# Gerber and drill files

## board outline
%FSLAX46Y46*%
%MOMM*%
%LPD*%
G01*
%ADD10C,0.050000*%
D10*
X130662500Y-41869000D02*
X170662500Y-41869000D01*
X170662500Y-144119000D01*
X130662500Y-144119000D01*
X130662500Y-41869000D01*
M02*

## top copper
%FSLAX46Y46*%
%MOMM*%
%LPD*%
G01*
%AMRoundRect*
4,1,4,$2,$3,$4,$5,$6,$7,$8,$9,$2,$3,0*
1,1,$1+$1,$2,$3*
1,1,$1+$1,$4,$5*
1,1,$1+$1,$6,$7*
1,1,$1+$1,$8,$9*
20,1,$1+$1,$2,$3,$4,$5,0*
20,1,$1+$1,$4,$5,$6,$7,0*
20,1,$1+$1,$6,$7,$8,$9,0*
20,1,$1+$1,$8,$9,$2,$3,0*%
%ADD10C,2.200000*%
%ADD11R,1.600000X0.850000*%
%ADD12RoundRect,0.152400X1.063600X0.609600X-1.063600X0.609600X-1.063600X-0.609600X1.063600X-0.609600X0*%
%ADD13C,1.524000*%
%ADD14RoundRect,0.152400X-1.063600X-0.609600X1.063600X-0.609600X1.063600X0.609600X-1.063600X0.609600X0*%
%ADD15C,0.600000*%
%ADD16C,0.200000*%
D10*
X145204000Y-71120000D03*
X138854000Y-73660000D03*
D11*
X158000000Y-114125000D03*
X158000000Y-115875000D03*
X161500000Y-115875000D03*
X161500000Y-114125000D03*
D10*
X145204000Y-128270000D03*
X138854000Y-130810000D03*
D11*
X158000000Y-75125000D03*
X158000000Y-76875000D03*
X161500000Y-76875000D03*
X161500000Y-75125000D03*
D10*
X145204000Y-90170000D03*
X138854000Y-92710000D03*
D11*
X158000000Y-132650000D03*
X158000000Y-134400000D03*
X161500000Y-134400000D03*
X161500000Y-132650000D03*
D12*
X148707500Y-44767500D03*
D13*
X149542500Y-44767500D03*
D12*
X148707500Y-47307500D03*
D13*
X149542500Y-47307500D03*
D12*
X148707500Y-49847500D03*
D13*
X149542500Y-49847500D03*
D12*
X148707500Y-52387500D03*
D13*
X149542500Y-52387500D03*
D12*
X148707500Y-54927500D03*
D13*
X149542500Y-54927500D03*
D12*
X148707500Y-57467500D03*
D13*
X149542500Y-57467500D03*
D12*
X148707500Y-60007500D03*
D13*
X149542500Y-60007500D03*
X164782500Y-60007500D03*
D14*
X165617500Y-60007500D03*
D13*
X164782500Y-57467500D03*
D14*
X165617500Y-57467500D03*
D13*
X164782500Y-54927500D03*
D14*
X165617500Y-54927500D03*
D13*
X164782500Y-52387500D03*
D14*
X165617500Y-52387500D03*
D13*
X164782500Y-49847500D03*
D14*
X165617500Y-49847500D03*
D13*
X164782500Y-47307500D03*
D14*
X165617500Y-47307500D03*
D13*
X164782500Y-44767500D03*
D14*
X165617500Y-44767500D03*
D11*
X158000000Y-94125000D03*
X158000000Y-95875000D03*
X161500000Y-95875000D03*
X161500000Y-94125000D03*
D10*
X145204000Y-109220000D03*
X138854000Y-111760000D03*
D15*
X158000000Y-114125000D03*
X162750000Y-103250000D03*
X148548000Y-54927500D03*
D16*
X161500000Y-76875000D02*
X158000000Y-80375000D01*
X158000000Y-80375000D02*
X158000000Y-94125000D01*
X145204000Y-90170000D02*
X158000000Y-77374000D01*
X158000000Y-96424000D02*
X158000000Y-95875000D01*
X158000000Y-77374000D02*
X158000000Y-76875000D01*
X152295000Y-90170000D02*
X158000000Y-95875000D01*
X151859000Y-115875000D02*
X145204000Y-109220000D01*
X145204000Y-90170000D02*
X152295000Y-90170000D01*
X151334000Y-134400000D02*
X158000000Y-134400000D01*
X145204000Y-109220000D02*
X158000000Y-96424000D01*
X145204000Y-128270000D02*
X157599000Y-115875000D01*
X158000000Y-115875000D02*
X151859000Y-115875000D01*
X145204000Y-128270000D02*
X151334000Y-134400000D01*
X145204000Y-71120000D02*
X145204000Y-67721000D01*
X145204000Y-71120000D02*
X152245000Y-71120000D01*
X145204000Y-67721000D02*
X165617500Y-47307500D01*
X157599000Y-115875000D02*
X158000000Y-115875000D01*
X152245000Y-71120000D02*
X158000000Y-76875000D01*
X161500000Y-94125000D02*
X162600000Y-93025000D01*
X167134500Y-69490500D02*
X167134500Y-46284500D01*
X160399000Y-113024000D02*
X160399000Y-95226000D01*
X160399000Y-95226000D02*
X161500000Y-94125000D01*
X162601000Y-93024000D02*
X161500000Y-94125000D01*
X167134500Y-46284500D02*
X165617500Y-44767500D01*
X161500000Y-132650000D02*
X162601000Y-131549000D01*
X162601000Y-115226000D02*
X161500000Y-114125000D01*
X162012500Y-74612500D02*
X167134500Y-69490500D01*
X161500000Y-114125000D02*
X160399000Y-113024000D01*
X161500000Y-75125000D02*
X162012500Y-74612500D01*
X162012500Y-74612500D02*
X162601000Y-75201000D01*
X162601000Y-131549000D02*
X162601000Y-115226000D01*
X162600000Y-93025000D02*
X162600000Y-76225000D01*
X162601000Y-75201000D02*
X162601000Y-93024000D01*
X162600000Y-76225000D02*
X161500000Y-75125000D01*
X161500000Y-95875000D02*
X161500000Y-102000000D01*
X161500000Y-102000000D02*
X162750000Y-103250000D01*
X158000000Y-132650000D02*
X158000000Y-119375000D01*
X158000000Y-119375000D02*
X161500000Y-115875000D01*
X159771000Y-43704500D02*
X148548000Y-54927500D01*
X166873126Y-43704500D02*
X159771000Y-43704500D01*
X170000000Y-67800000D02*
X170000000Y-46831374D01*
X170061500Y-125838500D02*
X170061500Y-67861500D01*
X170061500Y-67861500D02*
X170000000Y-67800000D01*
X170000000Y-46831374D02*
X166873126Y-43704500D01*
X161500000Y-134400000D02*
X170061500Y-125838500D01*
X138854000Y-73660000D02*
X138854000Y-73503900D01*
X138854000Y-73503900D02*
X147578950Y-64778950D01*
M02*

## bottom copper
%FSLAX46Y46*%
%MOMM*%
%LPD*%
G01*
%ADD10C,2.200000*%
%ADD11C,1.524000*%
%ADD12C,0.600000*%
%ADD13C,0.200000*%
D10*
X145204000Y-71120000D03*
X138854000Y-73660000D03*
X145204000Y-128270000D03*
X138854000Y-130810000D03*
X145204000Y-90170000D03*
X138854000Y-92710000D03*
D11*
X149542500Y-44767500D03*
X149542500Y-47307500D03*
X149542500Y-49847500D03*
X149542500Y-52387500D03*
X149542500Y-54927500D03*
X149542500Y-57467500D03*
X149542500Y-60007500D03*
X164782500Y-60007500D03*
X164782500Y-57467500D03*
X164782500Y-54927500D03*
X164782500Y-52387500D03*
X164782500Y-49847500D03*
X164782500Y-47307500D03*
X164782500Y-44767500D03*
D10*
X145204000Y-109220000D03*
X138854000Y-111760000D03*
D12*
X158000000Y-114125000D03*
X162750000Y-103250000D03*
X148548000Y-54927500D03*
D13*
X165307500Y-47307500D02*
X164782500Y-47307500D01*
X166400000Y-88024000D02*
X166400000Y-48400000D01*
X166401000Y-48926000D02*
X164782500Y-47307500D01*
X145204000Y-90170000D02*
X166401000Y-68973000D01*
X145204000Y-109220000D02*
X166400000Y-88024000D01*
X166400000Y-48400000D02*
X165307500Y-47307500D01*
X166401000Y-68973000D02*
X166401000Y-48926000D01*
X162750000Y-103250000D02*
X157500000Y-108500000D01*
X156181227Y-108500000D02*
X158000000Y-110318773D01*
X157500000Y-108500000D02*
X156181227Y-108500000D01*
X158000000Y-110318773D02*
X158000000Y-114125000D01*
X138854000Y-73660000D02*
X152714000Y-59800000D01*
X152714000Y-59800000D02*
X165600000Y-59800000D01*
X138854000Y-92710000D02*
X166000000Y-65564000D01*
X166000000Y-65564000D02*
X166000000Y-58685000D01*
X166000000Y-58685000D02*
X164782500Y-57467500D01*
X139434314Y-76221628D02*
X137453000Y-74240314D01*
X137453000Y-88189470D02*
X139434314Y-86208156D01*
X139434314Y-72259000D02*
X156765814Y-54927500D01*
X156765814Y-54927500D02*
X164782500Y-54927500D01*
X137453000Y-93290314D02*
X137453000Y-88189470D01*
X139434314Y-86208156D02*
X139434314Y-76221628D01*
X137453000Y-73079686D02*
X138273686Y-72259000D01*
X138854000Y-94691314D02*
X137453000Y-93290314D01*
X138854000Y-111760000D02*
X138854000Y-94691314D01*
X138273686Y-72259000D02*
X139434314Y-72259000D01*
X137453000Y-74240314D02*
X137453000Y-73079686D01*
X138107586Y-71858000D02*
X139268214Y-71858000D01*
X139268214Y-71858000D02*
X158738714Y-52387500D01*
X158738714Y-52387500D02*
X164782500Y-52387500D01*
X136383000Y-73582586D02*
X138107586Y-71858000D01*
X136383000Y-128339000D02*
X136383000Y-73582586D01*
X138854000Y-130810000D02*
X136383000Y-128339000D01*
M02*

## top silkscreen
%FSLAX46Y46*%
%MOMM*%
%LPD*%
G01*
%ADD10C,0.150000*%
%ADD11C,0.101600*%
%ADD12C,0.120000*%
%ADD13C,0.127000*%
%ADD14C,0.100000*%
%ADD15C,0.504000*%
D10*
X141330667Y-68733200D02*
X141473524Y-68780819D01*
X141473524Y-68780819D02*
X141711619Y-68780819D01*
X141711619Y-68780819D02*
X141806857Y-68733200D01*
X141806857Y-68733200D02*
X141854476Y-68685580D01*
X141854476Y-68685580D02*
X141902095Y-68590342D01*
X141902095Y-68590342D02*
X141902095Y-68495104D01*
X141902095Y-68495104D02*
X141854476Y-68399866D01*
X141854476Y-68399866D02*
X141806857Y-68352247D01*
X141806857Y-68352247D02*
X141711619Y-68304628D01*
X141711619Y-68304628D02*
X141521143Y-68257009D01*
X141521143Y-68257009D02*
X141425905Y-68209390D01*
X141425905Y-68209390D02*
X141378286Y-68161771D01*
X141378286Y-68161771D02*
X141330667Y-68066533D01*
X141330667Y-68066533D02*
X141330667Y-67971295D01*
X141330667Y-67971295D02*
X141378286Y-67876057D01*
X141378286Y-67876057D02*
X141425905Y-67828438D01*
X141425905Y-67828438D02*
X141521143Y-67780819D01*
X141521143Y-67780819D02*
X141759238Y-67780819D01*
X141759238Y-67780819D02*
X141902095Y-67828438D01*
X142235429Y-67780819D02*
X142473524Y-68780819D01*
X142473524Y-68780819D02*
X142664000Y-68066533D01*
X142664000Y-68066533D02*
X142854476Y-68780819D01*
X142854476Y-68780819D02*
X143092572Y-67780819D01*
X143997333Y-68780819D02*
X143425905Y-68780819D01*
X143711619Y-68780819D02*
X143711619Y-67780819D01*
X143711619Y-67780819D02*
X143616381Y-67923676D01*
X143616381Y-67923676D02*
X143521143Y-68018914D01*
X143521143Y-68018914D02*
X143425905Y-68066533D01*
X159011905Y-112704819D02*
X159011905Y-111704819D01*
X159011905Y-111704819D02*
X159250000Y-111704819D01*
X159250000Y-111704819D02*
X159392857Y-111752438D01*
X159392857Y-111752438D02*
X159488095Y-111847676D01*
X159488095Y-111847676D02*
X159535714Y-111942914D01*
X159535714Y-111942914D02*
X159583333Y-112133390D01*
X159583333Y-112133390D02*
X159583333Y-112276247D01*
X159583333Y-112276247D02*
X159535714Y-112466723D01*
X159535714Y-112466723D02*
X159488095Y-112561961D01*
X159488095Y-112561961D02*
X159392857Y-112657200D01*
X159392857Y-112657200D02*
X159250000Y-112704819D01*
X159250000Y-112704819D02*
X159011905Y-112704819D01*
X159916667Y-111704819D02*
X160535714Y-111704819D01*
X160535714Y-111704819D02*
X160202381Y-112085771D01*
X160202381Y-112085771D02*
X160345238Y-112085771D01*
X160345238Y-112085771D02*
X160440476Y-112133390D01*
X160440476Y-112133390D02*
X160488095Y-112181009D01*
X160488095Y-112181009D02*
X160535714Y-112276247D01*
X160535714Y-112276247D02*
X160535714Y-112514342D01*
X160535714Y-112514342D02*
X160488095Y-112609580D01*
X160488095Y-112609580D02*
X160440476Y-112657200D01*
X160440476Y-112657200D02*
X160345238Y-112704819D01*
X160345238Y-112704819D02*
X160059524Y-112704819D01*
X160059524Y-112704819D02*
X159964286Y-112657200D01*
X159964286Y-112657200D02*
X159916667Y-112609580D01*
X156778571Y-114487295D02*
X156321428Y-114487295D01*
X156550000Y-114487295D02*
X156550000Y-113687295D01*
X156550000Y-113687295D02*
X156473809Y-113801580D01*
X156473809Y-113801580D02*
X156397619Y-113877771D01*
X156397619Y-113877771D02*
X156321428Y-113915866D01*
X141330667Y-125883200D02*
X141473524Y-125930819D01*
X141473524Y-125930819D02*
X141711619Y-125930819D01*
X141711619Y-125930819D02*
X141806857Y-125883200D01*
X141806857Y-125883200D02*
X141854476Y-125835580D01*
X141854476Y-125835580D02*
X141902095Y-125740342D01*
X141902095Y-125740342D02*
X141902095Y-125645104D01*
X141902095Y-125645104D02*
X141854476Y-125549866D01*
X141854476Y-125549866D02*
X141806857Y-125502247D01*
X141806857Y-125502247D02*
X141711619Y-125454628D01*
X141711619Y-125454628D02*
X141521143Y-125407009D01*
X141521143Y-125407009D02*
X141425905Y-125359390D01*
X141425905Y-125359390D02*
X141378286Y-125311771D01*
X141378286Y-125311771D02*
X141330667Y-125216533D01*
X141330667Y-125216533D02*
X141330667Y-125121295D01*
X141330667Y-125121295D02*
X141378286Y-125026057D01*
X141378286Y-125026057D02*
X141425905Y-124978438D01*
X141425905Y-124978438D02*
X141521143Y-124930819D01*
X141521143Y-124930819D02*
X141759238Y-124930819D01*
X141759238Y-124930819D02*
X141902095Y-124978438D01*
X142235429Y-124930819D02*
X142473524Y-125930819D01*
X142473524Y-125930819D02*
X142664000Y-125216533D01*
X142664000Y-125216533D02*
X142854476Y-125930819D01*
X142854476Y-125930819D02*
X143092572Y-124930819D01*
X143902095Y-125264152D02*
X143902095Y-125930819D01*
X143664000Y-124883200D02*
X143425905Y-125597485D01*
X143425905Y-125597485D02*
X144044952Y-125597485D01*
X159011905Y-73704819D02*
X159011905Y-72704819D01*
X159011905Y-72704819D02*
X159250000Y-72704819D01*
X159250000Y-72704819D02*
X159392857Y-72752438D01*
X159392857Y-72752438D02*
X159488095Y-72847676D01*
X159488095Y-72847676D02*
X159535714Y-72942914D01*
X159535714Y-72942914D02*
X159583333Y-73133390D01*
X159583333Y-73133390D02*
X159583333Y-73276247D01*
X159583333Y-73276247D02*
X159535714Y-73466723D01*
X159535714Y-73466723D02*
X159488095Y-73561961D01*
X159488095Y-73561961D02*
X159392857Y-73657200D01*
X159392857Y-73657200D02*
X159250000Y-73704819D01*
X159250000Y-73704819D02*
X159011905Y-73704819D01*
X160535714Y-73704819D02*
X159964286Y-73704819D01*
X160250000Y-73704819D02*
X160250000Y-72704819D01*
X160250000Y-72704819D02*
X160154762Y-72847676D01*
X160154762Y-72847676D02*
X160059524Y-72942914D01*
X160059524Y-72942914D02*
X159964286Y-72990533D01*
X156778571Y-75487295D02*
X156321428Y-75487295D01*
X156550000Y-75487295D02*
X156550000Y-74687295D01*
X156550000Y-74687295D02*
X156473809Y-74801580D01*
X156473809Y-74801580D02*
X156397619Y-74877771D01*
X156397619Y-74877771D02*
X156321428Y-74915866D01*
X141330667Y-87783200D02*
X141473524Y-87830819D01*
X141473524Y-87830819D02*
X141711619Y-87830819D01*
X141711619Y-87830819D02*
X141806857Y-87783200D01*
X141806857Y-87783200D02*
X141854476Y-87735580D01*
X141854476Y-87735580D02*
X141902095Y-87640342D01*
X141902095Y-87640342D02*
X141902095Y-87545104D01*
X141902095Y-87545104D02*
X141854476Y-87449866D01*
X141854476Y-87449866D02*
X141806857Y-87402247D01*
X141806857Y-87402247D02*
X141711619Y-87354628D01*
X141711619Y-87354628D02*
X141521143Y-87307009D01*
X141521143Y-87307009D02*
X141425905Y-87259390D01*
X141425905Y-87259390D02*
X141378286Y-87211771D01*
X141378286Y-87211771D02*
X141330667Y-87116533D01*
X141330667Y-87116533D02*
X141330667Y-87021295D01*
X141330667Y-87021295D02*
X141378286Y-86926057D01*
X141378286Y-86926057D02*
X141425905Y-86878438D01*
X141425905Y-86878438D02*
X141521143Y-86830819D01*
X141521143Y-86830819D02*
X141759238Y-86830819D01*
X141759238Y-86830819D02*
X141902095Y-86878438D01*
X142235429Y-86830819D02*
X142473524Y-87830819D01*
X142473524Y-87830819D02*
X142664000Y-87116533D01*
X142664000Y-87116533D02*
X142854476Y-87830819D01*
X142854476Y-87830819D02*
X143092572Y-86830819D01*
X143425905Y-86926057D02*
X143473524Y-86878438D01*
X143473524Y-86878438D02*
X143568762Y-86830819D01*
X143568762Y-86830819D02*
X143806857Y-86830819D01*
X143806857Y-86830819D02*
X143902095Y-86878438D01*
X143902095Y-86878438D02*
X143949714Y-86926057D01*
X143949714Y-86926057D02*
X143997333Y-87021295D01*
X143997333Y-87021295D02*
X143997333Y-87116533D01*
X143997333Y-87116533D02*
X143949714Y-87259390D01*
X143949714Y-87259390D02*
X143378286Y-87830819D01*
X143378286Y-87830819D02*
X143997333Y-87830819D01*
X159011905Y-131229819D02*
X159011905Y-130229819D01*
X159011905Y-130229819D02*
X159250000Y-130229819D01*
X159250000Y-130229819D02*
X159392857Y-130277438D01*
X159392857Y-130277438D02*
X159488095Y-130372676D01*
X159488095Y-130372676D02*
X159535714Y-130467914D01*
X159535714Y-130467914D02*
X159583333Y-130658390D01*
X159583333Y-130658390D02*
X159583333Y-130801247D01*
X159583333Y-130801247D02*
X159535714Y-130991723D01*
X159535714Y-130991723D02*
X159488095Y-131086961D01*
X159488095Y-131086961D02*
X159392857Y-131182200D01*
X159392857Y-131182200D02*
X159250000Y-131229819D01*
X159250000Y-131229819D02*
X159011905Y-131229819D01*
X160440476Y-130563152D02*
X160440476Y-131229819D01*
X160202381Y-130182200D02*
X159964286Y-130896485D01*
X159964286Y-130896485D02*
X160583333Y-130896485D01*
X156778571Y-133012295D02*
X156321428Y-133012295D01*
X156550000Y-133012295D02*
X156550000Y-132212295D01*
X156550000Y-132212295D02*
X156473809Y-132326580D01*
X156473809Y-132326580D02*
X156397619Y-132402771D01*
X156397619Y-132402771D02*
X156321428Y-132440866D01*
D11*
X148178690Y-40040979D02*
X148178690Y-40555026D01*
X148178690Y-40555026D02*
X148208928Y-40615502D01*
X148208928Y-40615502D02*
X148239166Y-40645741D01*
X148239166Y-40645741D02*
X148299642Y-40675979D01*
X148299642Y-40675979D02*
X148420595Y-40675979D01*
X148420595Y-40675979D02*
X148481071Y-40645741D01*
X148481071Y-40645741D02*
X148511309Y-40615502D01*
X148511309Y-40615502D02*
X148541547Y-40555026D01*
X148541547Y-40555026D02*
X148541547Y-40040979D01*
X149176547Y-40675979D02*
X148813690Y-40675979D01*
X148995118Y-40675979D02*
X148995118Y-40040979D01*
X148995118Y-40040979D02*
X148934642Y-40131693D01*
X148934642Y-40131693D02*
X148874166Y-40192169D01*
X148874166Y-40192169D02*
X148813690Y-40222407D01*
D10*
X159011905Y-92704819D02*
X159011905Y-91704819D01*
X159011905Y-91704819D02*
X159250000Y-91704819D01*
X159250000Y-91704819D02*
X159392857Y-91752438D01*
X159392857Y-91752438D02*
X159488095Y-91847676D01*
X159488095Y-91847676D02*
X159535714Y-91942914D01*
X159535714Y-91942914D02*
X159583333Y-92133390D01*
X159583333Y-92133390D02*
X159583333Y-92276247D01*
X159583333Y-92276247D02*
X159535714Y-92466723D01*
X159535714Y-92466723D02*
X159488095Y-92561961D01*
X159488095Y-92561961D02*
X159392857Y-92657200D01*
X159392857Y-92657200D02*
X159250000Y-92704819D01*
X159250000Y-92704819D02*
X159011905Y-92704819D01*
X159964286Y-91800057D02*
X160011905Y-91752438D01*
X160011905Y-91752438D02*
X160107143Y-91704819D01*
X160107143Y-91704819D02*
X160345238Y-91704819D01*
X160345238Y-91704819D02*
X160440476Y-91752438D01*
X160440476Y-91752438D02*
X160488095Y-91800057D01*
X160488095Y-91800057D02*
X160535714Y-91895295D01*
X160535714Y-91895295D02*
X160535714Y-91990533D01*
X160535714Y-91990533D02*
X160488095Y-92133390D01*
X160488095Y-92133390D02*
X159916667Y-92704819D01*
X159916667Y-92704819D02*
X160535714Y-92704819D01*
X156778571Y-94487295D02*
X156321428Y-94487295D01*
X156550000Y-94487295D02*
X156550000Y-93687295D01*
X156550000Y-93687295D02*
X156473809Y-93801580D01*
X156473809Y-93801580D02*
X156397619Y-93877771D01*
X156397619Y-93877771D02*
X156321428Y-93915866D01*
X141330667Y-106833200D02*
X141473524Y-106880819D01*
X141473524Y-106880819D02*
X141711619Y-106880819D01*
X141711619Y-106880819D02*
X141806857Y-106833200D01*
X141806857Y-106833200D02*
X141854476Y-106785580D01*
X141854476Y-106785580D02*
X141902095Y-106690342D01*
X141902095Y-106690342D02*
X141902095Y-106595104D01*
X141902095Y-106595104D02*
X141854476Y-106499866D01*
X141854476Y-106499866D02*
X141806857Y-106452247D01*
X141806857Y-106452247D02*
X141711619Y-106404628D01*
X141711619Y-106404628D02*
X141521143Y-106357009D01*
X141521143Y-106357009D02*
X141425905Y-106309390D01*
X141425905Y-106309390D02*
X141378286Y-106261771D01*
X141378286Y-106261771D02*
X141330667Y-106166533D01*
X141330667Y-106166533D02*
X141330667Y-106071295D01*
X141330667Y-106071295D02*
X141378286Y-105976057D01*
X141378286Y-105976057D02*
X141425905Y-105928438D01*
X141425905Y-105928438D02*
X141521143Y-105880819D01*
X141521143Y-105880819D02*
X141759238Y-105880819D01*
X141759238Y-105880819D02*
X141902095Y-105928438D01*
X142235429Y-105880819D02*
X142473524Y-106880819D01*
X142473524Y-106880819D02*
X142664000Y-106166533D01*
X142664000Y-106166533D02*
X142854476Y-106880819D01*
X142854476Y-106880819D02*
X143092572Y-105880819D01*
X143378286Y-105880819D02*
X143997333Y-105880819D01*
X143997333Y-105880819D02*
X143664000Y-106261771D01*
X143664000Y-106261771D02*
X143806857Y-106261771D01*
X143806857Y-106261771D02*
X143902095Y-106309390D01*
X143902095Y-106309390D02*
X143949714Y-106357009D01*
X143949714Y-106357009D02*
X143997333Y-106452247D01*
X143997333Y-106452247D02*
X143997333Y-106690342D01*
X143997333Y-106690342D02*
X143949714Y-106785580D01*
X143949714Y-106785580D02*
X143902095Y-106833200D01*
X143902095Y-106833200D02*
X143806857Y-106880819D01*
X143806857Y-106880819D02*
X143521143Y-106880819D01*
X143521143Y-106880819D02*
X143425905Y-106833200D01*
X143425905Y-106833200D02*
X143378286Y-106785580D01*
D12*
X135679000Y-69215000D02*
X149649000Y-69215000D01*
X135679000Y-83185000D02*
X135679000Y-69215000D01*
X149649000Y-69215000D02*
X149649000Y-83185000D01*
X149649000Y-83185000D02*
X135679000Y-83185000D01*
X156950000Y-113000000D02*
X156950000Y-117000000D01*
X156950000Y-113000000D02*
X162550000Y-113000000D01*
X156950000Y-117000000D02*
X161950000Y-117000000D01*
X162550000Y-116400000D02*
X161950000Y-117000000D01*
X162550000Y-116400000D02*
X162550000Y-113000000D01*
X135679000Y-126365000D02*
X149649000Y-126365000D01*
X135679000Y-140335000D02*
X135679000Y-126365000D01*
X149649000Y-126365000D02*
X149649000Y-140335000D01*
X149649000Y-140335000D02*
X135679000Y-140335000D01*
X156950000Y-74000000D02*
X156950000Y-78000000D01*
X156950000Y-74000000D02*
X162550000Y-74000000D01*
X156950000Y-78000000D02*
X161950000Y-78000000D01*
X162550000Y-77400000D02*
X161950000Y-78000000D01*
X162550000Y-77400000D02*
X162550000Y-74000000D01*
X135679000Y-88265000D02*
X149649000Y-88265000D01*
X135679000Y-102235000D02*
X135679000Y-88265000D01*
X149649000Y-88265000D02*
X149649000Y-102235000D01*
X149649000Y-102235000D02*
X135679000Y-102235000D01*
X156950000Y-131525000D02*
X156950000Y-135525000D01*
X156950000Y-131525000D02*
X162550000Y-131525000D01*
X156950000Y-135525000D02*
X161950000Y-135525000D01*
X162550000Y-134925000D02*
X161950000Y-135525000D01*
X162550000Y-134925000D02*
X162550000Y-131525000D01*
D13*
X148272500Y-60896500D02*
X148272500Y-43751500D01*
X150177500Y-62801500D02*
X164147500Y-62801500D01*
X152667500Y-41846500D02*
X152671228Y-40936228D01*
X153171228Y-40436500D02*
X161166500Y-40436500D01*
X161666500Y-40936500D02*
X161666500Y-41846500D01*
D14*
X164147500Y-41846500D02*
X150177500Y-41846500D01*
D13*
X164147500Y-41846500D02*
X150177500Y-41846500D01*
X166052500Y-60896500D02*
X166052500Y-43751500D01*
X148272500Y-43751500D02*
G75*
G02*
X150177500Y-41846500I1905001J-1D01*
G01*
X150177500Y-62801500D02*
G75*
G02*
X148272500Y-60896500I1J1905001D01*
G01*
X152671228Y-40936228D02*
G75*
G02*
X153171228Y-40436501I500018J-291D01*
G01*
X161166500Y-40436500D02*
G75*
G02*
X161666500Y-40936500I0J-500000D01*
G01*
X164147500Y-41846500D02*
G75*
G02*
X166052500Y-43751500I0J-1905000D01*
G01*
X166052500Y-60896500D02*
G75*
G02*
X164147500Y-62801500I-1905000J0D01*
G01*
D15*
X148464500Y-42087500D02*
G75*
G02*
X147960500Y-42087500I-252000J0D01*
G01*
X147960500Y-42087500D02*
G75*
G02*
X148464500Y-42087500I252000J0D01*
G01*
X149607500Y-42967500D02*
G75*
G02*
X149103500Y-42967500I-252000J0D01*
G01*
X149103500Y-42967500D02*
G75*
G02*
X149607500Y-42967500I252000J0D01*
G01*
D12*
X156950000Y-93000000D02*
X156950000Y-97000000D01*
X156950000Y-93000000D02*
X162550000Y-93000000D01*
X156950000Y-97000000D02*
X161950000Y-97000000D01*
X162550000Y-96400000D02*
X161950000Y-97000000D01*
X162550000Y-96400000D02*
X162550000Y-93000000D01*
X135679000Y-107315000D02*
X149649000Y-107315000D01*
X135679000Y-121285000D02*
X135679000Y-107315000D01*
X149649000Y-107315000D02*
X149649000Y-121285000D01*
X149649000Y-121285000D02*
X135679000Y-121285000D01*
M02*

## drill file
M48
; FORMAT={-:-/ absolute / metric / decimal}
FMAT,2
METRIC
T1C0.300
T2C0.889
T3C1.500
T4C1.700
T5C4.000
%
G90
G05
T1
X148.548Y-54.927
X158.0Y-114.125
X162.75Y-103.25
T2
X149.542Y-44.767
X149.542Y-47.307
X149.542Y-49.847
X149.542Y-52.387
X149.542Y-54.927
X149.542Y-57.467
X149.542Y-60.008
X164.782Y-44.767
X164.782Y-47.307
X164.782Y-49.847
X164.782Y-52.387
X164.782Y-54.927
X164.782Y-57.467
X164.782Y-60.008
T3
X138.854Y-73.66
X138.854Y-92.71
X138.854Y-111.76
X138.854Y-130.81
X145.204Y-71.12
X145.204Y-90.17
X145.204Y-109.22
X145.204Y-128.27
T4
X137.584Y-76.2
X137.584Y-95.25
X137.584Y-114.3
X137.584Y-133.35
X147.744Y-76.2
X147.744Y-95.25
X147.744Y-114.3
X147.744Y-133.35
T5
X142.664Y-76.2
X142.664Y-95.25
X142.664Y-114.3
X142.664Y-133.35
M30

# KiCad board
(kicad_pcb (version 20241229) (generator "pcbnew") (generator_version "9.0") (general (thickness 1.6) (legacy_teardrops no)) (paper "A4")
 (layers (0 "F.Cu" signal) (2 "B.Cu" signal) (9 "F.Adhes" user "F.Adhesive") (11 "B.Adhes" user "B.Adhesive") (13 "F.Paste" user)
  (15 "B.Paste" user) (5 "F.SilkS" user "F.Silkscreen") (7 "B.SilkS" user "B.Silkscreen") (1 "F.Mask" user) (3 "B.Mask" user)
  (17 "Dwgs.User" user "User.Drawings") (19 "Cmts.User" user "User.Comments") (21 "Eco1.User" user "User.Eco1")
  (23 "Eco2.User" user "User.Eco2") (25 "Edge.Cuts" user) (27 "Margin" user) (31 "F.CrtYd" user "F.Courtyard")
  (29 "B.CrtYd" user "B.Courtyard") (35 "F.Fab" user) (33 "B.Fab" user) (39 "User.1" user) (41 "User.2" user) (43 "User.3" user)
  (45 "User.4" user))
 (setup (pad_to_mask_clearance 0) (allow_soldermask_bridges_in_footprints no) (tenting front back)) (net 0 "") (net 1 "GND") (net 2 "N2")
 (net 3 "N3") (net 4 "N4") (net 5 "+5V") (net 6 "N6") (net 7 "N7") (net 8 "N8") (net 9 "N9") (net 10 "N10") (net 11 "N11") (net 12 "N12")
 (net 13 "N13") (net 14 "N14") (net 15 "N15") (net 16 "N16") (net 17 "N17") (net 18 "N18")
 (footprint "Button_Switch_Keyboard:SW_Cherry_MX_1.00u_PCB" (layer "F.Cu") (at 145.204 71.12)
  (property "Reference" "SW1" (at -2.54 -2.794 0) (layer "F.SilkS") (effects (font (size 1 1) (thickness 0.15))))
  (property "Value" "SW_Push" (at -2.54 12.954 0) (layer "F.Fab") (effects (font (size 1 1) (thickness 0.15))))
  (fp_line (start -9.525 -1.905) (end 4.445 -1.905) (stroke (width 0.12) (type solid)) (layer "F.SilkS"))
  (fp_line (start -9.525 12.065) (end -9.525 -1.905) (stroke (width 0.12) (type solid)) (layer "F.SilkS"))
  (fp_line (start 4.445 -1.905) (end 4.445 12.065) (stroke (width 0.12) (type solid)) (layer "F.SilkS"))
  (fp_line (start 4.445 12.065) (end -9.525 12.065) (stroke (width 0.12) (type solid)) (layer "F.SilkS"))
  (pad "" np_thru_hole circle (at -7.62 5.08) (size 1.7 1.7) (drill 1.7) (layers "*.Cu" "*.Mask"))
  (pad "" np_thru_hole circle (at -2.54 5.08) (size 4 4) (drill 4) (layers "*.Cu" "*.Mask"))
  (pad "" np_thru_hole circle (at 2.54 5.08) (size 1.7 1.7) (drill 1.7) (layers "*.Cu" "*.Mask"))
  (pad "1" thru_hole circle (at 0 0) (size 2.2 2.2) (drill 1.5) (layers "*.Cu" "*.Mask") (remove_unused_layers no) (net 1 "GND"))
  (pad "2" thru_hole circle (at -6.35 2.54) (size 2.2 2.2) (drill 1.5) (layers "*.Cu" "*.Mask") (remove_unused_layers no) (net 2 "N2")))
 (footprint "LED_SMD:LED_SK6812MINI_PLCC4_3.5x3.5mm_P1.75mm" (layer "F.Cu") (at 159.75 115)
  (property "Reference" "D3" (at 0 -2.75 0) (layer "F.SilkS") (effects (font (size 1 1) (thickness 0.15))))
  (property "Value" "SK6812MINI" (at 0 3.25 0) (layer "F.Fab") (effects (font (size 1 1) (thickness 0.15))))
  (fp_line (start -2.8 -2) (end -2.8 2) (stroke (width 0.12) (type default)) (layer "F.SilkS"))
  (fp_line (start -2.8 -2) (end 2.8 -2) (stroke (width 0.12) (type solid)) (layer "F.SilkS"))
  (fp_line (start -2.8 2) (end 2.2 2) (stroke (width 0.12) (type solid)) (layer "F.SilkS"))
  (fp_line (start 2.8 1.4) (end 2.2 2) (stroke (width 0.12) (type default)) (layer "F.SilkS"))
  (fp_line (start 2.8 1.4) (end 2.8 -2) (stroke (width 0.12) (type solid)) (layer "F.SilkS"))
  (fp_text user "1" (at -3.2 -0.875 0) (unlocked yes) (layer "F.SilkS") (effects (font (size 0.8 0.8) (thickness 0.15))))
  (pad "1" smd rect (at -1.75 -0.875) (size 1.6 0.85) (layers "F.Cu" "F.Mask" "F.Paste") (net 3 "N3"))
  (pad "2" smd rect (at -1.75 0.875) (size 1.6 0.85) (layers "F.Cu" "F.Mask" "F.Paste") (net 1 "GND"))
  (pad "3" smd rect (at 1.75 0.875) (size 1.6 0.85) (layers "F.Cu" "F.Mask" "F.Paste") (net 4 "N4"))
  (pad "4" smd rect (at 1.75 -0.875) (size 1.6 0.85) (layers "F.Cu" "F.Mask" "F.Paste") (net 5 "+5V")))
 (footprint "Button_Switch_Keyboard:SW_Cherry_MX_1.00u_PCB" (layer "F.Cu") (at 145.204 128.27)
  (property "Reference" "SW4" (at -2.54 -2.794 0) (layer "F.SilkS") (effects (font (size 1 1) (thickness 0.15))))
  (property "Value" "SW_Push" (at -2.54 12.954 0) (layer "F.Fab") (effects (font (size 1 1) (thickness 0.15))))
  (fp_line (start -9.525 -1.905) (end 4.445 -1.905) (stroke (width 0.12) (type solid)) (layer "F.SilkS"))
  (fp_line (start -9.525 12.065) (end -9.525 -1.905) (stroke (width 0.12) (type solid)) (layer "F.SilkS"))
  (fp_line (start 4.445 -1.905) (end 4.445 12.065) (stroke (width 0.12) (type solid)) (layer "F.SilkS"))
  (fp_line (start 4.445 12.065) (end -9.525 12.065) (stroke (width 0.12) (type solid)) (layer "F.SilkS"))
  (pad "" np_thru_hole circle (at -7.62 5.08) (size 1.7 1.7) (drill 1.7) (layers "*.Cu" "*.Mask"))
  (pad "" np_thru_hole circle (at -2.54 5.08) (size 4 4) (drill 4) (layers "*.Cu" "*.Mask"))
  (pad "" np_thru_hole circle (at 2.54 5.08) (size 1.7 1.7) (drill 1.7) (layers "*.Cu" "*.Mask"))
  (pad "1" thru_hole circle (at 0 0) (size 2.2 2.2) (drill 1.5) (layers "*.Cu" "*.Mask") (remove_unused_layers no) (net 1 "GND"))
  (pad "2" thru_hole circle (at -6.35 2.54) (size 2.2 2.2) (drill 1.5) (layers "*.Cu" "*.Mask") (remove_unused_layers no) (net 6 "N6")))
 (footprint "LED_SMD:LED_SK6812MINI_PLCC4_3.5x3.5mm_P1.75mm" (layer "F.Cu") (at 159.75 76)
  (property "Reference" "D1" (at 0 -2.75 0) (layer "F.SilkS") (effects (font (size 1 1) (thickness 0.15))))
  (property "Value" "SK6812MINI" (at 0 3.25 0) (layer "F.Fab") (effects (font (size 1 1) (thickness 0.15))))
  (fp_line (start -2.8 -2) (end -2.8 2) (stroke (width 0.12) (type default)) (layer "F.SilkS"))
  (fp_line (start -2.8 -2) (end 2.8 -2) (stroke (width 0.12) (type solid)) (layer "F.SilkS"))
  (fp_line (start -2.8 2) (end 2.2 2) (stroke (width 0.12) (type solid)) (layer "F.SilkS"))
  (fp_line (start 2.8 1.4) (end 2.2 2) (stroke (width 0.12) (type default)) (layer "F.SilkS"))
  (fp_line (start 2.8 1.4) (end 2.8 -2) (stroke (width 0.12) (type solid)) (layer "F.SilkS"))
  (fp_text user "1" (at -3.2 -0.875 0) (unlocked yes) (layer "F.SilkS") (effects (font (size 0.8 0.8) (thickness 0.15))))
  (pad "1" smd rect (at -1.75 -0.875) (size 1.6 0.85) (layers "F.Cu" "F.Mask" "F.Paste") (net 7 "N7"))
  (pad "2" smd rect (at -1.75 0.875) (size 1.6 0.85) (layers "F.Cu" "F.Mask" "F.Paste") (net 1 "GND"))
  (pad "3" smd rect (at 1.75 0.875) (size 1.6 0.85) (layers "F.Cu" "F.Mask" "F.Paste") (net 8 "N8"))
  (pad "4" smd rect (at 1.75 -0.875) (size 1.6 0.85) (layers "F.Cu" "F.Mask" "F.Paste") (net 5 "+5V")))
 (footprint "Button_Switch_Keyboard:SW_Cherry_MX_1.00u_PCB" (layer "F.Cu") (at 145.204 90.17)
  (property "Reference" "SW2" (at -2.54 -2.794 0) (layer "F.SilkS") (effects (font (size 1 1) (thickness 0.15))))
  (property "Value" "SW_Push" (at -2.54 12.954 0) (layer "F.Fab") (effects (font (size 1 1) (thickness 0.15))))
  (fp_line (start -9.525 -1.905) (end 4.445 -1.905) (stroke (width 0.12) (type solid)) (layer "F.SilkS"))
  (fp_line (start -9.525 12.065) (end -9.525 -1.905) (stroke (width 0.12) (type solid)) (layer "F.SilkS"))
  (fp_line (start 4.445 -1.905) (end 4.445 12.065) (stroke (width 0.12) (type solid)) (layer "F.SilkS"))
  (fp_line (start 4.445 12.065) (end -9.525 12.065) (stroke (width 0.12) (type solid)) (layer "F.SilkS"))
  (pad "" np_thru_hole circle (at -7.62 5.08) (size 1.7 1.7) (drill 1.7) (layers "*.Cu" "*.Mask"))
  (pad "" np_thru_hole circle (at -2.54 5.08) (size 4 4) (drill 4) (layers "*.Cu" "*.Mask"))
  (pad "" np_thru_hole circle (at 2.54 5.08) (size 1.7 1.7) (drill 1.7) (layers "*.Cu" "*.Mask"))
  (pad "1" thru_hole circle (at 0 0) (size 2.2 2.2) (drill 1.5) (layers "*.Cu" "*.Mask") (remove_unused_layers no) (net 1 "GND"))
  (pad "2" thru_hole circle (at -6.35 2.54) (size 2.2 2.2) (drill 1.5) (layers "*.Cu" "*.Mask") (remove_unused_layers no) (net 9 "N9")))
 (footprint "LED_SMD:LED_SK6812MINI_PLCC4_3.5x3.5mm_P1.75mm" (layer "F.Cu") (at 159.75 133.525)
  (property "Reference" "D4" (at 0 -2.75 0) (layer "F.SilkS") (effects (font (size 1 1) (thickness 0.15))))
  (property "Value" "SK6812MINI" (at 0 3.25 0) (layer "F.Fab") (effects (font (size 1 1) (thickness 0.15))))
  (fp_line (start -2.8 -2) (end -2.8 2) (stroke (width 0.12) (type default)) (layer "F.SilkS"))
  (fp_line (start -2.8 -2) (end 2.8 -2) (stroke (width 0.12) (type solid)) (layer "F.SilkS"))
  (fp_line (start -2.8 2) (end 2.2 2) (stroke (width 0.12) (type solid)) (layer "F.SilkS"))
  (fp_line (start 2.8 1.4) (end 2.2 2) (stroke (width 0.12) (type default)) (layer "F.SilkS"))
  (fp_line (start 2.8 1.4) (end 2.8 -2) (stroke (width 0.12) (type solid)) (layer "F.SilkS"))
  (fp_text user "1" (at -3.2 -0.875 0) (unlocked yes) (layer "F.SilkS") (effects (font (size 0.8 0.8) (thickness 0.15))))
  (pad "1" smd rect (at -1.75 -0.875) (size 1.6 0.85) (layers "F.Cu" "F.Mask" "F.Paste") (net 4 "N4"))
  (pad "2" smd rect (at -1.75 0.875) (size 1.6 0.85) (layers "F.Cu" "F.Mask" "F.Paste") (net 1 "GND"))
  (pad "3" smd rect (at 1.75 0.875) (size 1.6 0.85) (layers "F.Cu" "F.Mask" "F.Paste") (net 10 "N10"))
  (pad "4" smd rect (at 1.75 -0.875) (size 1.6 0.85) (layers "F.Cu" "F.Mask" "F.Paste") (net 5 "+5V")))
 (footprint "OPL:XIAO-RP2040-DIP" (layer "F.Cu") (at 157.1625 52.3875)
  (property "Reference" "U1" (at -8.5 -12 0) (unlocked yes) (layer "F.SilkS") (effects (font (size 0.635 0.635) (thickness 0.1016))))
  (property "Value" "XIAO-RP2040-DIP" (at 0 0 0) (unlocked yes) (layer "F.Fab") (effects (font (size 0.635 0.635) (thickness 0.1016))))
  (fp_line (start -8.89 8.509) (end -8.89 -8.636) (stroke (width 0.127) (type solid)) (layer "F.SilkS"))
  (fp_line (start -6.985 10.414) (end 6.985 10.414) (stroke (width 0.127) (type solid)) (layer "F.SilkS"))
  (fp_line (start -4.495 -10.541) (end -4.491272 -11.451272) (stroke (width 0.127) (type solid)) (layer "F.SilkS"))
  (fp_line (start -3.991272 -11.951) (end 4.004 -11.951) (stroke (width 0.127) (type solid)) (layer "F.SilkS"))
  (fp_line (start 4.504 -11.451) (end 4.504 -10.541) (stroke (width 0.127) (type solid)) (layer "F.SilkS"))
  (fp_line (start 6.985 -10.541) (end -6.985 -10.541) (stroke (width 0.1) (type solid)) (layer "F.SilkS"))
  (fp_line (start 6.985 -10.541) (end -6.985 -10.541) (stroke (width 0.127) (type solid)) (layer "F.SilkS"))
  (fp_line (start 8.89 8.509) (end 8.89 -8.636) (stroke (width 0.127) (type solid)) (layer "F.SilkS"))
  (fp_arc (start -8.89 -8.636) (mid -8.332038 -9.983038) (end -6.985 -10.541) (stroke (width 0.127) (type solid)) (layer "F.SilkS"))
  (fp_arc (start -6.985 10.414) (mid -8.332038 9.856038) (end -8.89 8.509) (stroke (width 0.127) (type solid)) (layer "F.SilkS"))
  (fp_arc (start -4.491272 -11.451272) (mid -4.344728 -11.80464) (end -3.991272 -11.951) (stroke (width 0.127) (type default))
   (layer "F.SilkS"))
  (fp_arc (start 4.004 -11.951) (mid 4.357553 -11.804553) (end 4.504 -11.451) (stroke (width 0.127) (type default)) (layer "F.SilkS"))
  (fp_arc (start 6.985 -10.541) (mid 8.332038 -9.983038) (end 8.89 -8.636) (stroke (width 0.127) (type solid)) (layer "F.SilkS"))
  (fp_arc (start 8.89 8.509) (mid 8.332038 9.856038) (end 6.985 10.414) (stroke (width 0.127) (type solid)) (layer "F.SilkS"))
  (fp_circle (center -8.95 -10.3) (end -8.95 -10.554) (stroke (width 0.5) (type solid)) (fill yes) (layer "F.SilkS"))
  (fp_circle (center -7.807 -9.42) (end -7.807 -9.674) (stroke (width 0.5) (type solid)) (fill yes) (layer "F.SilkS"))
  (pad "1" smd roundrect (at -8.455 -7.62 180) (size 2.432 1.524) (layers "F.Cu" "F.Mask") (roundrect_rratio 0.1) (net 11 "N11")
   (thermal_bridge_angle 45))
  (pad "1" thru_hole circle (at -7.62 -7.62 180) (size 1.524 1.524) (drill 0.889) (layers "*.Cu" "*.Mask") (remove_unused_layers no)
   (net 11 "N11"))
  (pad "2" smd roundrect (at -8.455 -5.08 180) (size 2.432 1.524) (layers "F.Cu" "F.Mask") (roundrect_rratio 0.1) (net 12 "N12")
   (thermal_bridge_angle 45))
  (pad "2" thru_hole circle (at -7.62 -5.08 180) (size 1.524 1.524) (drill 0.889) (layers "*.Cu" "*.Mask") (remove_unused_layers no)
   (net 12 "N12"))
  (pad "3" smd roundrect (at -8.455 -2.54 180) (size 2.432 1.524) (layers "F.Cu" "F.Mask") (roundrect_rratio 0.1) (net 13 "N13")
   (thermal_bridge_angle 45))
  (pad "3" thru_hole circle (at -7.62 -2.54 180) (size 1.524 1.524) (drill 0.889) (layers "*.Cu" "*.Mask") (remove_unused_layers no)
   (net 13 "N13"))
  (pad "4" smd roundrect (at -8.455 0 180) (size 2.432 1.524) (layers "F.Cu" "F.Mask") (roundrect_rratio 0.1) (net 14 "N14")
   (thermal_bridge_angle 45))
  (pad "4" thru_hole circle (at -7.62 0 180) (size 1.524 1.524) (drill 0.889) (layers "*.Cu" "*.Mask") (remove_unused_layers no)
   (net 14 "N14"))
  (pad "5" smd roundrect (at -8.455 2.54 180) (size 2.432 1.524) (layers "F.Cu" "F.Mask") (roundrect_rratio 0.1) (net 10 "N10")
   (thermal_bridge_angle 45))
  (pad "5" thru_hole circle (at -7.62 2.54 180) (size 1.524 1.524) (drill 0.889) (layers "*.Cu" "*.Mask") (remove_unused_layers no)
   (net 10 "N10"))
  (pad "6" smd roundrect (at -8.455 5.08 180) (size 2.432 1.524) (layers "F.Cu" "F.Mask") (roundrect_rratio 0.1) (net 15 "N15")
   (thermal_bridge_angle 45))
  (pad "6" thru_hole circle (at -7.62 5.08 180) (size 1.524 1.524) (drill 0.889) (layers "*.Cu" "*.Mask") (remove_unused_layers no)
   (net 15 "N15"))
  (pad "7" smd roundrect (at -8.455 7.62 180) (size 2.432 1.524) (layers "F.Cu" "F.Mask") (roundrect_rratio 0.1) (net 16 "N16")
   (thermal_bridge_angle 45))
  (pad "7" thru_hole circle (at -7.62 7.62 180) (size 1.524 1.524) (drill 0.889) (layers "*.Cu" "*.Mask") (remove_unused_layers no)
   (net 16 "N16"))
  (pad "8" thru_hole circle (at 7.62 7.62) (size 1.524 1.524) (drill 0.889) (layers "*.Cu" "*.Mask") (remove_unused_layers no) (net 2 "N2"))
  (pad "8" smd roundrect (at 8.455 7.62) (size 2.432 1.524) (layers "F.Cu" "F.Mask") (roundrect_rratio 0.1) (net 2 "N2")
   (thermal_bridge_angle 45))
  (pad "9" thru_hole circle (at 7.62 5.08) (size 1.524 1.524) (drill 0.889) (layers "*.Cu" "*.Mask") (remove_unused_layers no) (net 9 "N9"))
  (pad "9" smd roundrect (at 8.455 5.08) (size 2.432 1.524) (layers "F.Cu" "F.Mask") (roundrect_rratio 0.1) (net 9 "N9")
   (thermal_bridge_angle 45))
  (pad "10" thru_hole circle (at 7.62 2.54) (size 1.524 1.524) (drill 0.889) (layers "*.Cu" "*.Mask") (remove_unused_layers no)
   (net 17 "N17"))
  (pad "10" smd roundrect (at 8.455 2.54) (size 2.432 1.524) (layers "F.Cu" "F.Mask") (roundrect_rratio 0.1) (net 17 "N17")
   (thermal_bridge_angle 45))
  (pad "11" thru_hole circle (at 7.62 0) (size 1.524 1.524) (drill 0.889) (layers "*.Cu" "*.Mask") (remove_unused_layers no) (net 6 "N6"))
  (pad "11" smd roundrect (at 8.455 0) (size 2.432 1.524) (layers "F.Cu" "F.Mask") (roundrect_rratio 0.1) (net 6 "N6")
   (thermal_bridge_angle 45))
  (pad "12" thru_hole circle (at 7.62 -2.54) (size 1.524 1.524) (drill 0.889) (layers "*.Cu" "*.Mask") (remove_unused_layers no)
   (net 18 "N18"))
  (pad "12" smd roundrect (at 8.455 -2.54) (size 2.432 1.524) (layers "F.Cu" "F.Mask") (roundrect_rratio 0.1) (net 18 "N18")
   (thermal_bridge_angle 45))
  (pad "13" thru_hole circle (at 7.62 -5.08) (size 1.524 1.524) (drill 0.889) (layers "*.Cu" "*.Mask") (remove_unused_layers no)
   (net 1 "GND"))
  (pad "13" smd roundrect (at 8.455 -5.08) (size 2.432 1.524) (layers "F.Cu" "F.Mask") (roundrect_rratio 0.1) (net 1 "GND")
   (thermal_bridge_angle 45))
  (pad "14" thru_hole circle (at 7.62 -7.62) (size 1.524 1.524) (drill 0.889) (layers "*.Cu" "*.Mask") (remove_unused_layers no)
   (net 5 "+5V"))
  (pad "14" smd roundrect (at 8.455 -7.62) (size 2.432 1.524) (layers "F.Cu" "F.Mask") (roundrect_rratio 0.1) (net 5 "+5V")
   (thermal_bridge_angle 45)))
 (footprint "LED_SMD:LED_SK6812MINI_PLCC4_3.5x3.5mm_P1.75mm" (layer "F.Cu") (at 159.75 95)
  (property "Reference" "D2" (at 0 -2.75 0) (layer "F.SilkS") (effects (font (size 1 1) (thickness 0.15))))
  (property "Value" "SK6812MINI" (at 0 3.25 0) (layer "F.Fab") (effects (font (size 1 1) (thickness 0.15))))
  (fp_line (start -2.8 -2) (end -2.8 2) (stroke (width 0.12) (type default)) (layer "F.SilkS"))
  (fp_line (start -2.8 -2) (end 2.8 -2) (stroke (width 0.12) (type solid)) (layer "F.SilkS"))
  (fp_line (start -2.8 2) (end 2.2 2) (stroke (width 0.12) (type solid)) (layer "F.SilkS"))
  (fp_line (start 2.8 1.4) (end 2.2 2) (stroke (width 0.12) (type default)) (layer "F.SilkS"))
  (fp_line (start 2.8 1.4) (end 2.8 -2) (stroke (width 0.12) (type solid)) (layer "F.SilkS"))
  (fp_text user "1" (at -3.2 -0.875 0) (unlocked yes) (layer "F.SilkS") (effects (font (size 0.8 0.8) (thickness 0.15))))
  (pad "1" smd rect (at -1.75 -0.875) (size 1.6 0.85) (layers "F.Cu" "F.Mask" "F.Paste") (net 8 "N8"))
  (pad "2" smd rect (at -1.75 0.875) (size 1.6 0.85) (layers "F.Cu" "F.Mask" "F.Paste") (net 1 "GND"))
  (pad "3" smd rect (at 1.75 0.875) (size 1.6 0.85) (layers "F.Cu" "F.Mask" "F.Paste") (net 3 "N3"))
  (pad "4" smd rect (at 1.75 -0.875) (size 1.6 0.85) (layers "F.Cu" "F.Mask" "F.Paste") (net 5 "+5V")))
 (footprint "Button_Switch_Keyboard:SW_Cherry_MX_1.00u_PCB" (layer "F.Cu") (at 145.204 109.22)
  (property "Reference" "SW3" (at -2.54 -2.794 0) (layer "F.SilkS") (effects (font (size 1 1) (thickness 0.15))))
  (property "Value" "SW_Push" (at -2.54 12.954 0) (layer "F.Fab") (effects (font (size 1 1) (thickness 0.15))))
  (fp_line (start -9.525 -1.905) (end 4.445 -1.905) (stroke (width 0.12) (type solid)) (layer "F.SilkS"))
  (fp_line (start -9.525 12.065) (end -9.525 -1.905) (stroke (width 0.12) (type solid)) (layer "F.SilkS"))
  (fp_line (start 4.445 -1.905) (end 4.445 12.065) (stroke (width 0.12) (type solid)) (layer "F.SilkS"))
  (fp_line (start 4.445 12.065) (end -9.525 12.065) (stroke (width 0.12) (type solid)) (layer "F.SilkS"))
  (pad "" np_thru_hole circle (at -7.62 5.08) (size 1.7 1.7) (drill 1.7) (layers "*.Cu" "*.Mask"))
  (pad "" np_thru_hole circle (at -2.54 5.08) (size 4 4) (drill 4) (layers "*.Cu" "*.Mask"))
  (pad "" np_thru_hole circle (at 2.54 5.08) (size 1.7 1.7) (drill 1.7) (layers "*.Cu" "*.Mask"))
  (pad "1" thru_hole circle (at 0 0) (size 2.2 2.2) (drill 1.5) (layers "*.Cu" "*.Mask") (remove_unused_layers no) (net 1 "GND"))
  (pad "2" thru_hole circle (at -6.35 2.54) (size 2.2 2.2) (drill 1.5) (layers "*.Cu" "*.Mask") (remove_unused_layers no) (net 17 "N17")))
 (gr_rect (start 130.6625 41.869) (end 170.6625 144.119) (stroke (width 0.05) (type default)) (fill no) (layer "Edge.Cuts"))
 (segment (start 161.5 76.875) (end 158 80.375) (width 0.2) (layer "F.Cu") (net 8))
 (segment (start 158 80.375) (end 158 94.125) (width 0.2) (layer "F.Cu") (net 8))
 (segment (start 145.204 90.17) (end 158 77.374) (width 0.2) (layer "F.Cu") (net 1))
 (segment (start 158 96.424) (end 158 95.875) (width 0.2) (layer "F.Cu") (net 1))
 (segment (start 158 77.374) (end 158 76.875) (width 0.2) (layer "F.Cu") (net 1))
 (segment (start 152.295 90.17) (end 158 95.875) (width 0.2) (layer "F.Cu") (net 1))
 (segment (start 151.859 115.875) (end 145.204 109.22) (width 0.2) (layer "F.Cu") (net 1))
 (segment (start 145.204 90.17) (end 152.295 90.17) (width 0.2) (layer "F.Cu") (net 1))
 (segment (start 151.334 134.4) (end 158 134.4) (width 0.2) (layer "F.Cu") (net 1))
 (segment (start 145.204 109.22) (end 158 96.424) (width 0.2) (layer "F.Cu") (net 1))
 (segment (start 145.204 128.27) (end 157.599 115.875) (width 0.2) (layer "F.Cu") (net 1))
 (segment (start 158 115.875) (end 151.859 115.875) (width 0.2) (layer "F.Cu") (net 1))
 (segment (start 145.204 128.27) (end 151.334 134.4) (width 0.2) (layer "F.Cu") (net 1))
 (segment (start 145.204 71.12) (end 145.204 67.721) (width 0.2) (layer "F.Cu") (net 1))
 (segment (start 145.204 71.12) (end 152.245 71.12) (width 0.2) (layer "F.Cu") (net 1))
 (segment (start 145.204 67.721) (end 165.6175 47.3075) (width 0.2) (layer "F.Cu") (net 1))
 (segment (start 157.599 115.875) (end 158 115.875) (width 0.2) (layer "F.Cu") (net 1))
 (segment (start 152.245 71.12) (end 158 76.875) (width 0.2) (layer "F.Cu") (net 1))
 (segment (start 165.3075 47.3075) (end 164.7825 47.3075) (width 0.2) (layer "B.Cu") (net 1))
 (segment (start 166.4 88.024) (end 166.4 48.4) (width 0.2) (layer "B.Cu") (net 1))
 (segment (start 166.401 48.926) (end 164.7825 47.3075) (width 0.2) (layer "B.Cu") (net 1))
 (segment (start 145.204 90.17) (end 166.401 68.973) (width 0.2) (layer "B.Cu") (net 1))
 (segment (start 145.204 109.22) (end 166.4 88.024) (width 0.2) (layer "B.Cu") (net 1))
 (segment (start 166.4 48.4) (end 165.3075 47.3075) (width 0.2) (layer "B.Cu") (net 1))
 (segment (start 166.401 68.973) (end 166.401 48.926) (width 0.2) (layer "B.Cu") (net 1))
 (segment (start 161.5 94.125) (end 162.6 93.025) (width 0.2) (layer "F.Cu") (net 5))
 (segment (start 167.1345 69.4905) (end 167.1345 46.2845) (width 0.2) (layer "F.Cu") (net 5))
 (segment (start 160.399 113.024) (end 160.399 95.226) (width 0.2) (layer "F.Cu") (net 5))
 (segment (start 160.399 95.226) (end 161.5 94.125) (width 0.2) (layer "F.Cu") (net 5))
 (segment (start 162.601 93.024) (end 161.5 94.125) (width 0.2) (layer "F.Cu") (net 5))
 (segment (start 167.1345 46.2845) (end 165.6175 44.7675) (width 0.2) (layer "F.Cu") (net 5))
 (segment (start 161.5 132.65) (end 162.601 131.549) (width 0.2) (layer "F.Cu") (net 5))
 (segment (start 162.601 115.226) (end 161.5 114.125) (width 0.2) (layer "F.Cu") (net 5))
 (segment (start 162.0125 74.6125) (end 167.1345 69.4905) (width 0.2) (layer "F.Cu") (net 5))
 (segment (start 161.5 114.125) (end 160.399 113.024) (width 0.2) (layer "F.Cu") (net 5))
 (segment (start 161.5 75.125) (end 162.0125 74.6125) (width 0.2) (layer "F.Cu") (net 5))
 (segment (start 162.0125 74.6125) (end 162.601 75.201) (width 0.2) (layer "F.Cu") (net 5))
 (segment (start 162.601 131.549) (end 162.601 115.226) (width 0.2) (layer "F.Cu") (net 5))
 (segment (start 162.6 93.025) (end 162.6 76.225) (width 0.2) (layer "F.Cu") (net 5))
 (segment (start 162.601 75.201) (end 162.601 93.024) (width 0.2) (layer "F.Cu") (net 5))
 (segment (start 162.6 76.225) (end 161.5 75.125) (width 0.2) (layer "F.Cu") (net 5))
 (segment (start 161.5 95.875) (end 161.5 102) (width 0.2) (layer "F.Cu") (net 3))
 (segment (start 161.5 102) (end 162.75 103.25) (width 0.2) (layer "F.Cu") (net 3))
 (via (at 158 114.125) (size 0.6) (drill 0.3) (layers "F.Cu" "B.Cu") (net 3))
 (via (at 162.75 103.25) (size 0.6) (drill 0.3) (layers "F.Cu" "B.Cu") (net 3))
 (segment (start 162.75 103.25) (end 157.5 108.5) (width 0.2) (layer "B.Cu") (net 3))
 (segment (start 156.181227 108.5) (end 158 110.318773) (width 0.2) (layer "B.Cu") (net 3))
 (segment (start 157.5 108.5) (end 156.181227 108.5) (width 0.2) (layer "B.Cu") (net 3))
 (segment (start 158 110.318773) (end 158 114.125) (width 0.2) (layer "B.Cu") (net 3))
 (segment (start 158 132.65) (end 158 119.375) (width 0.2) (layer "F.Cu") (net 4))
 (segment (start 158 119.375) (end 161.5 115.875) (width 0.2) (layer "F.Cu") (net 4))
 (segment (start 159.771 43.7045) (end 148.548 54.9275) (width 0.2) (layer "F.Cu") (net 10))
 (segment (start 166.873126 43.7045) (end 159.771 43.7045) (width 0.2) (layer "F.Cu") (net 10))
 (segment (start 170 67.8) (end 170 46.831374) (width 0.2) (layer "F.Cu") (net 10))
 (segment (start 170.0615 125.8385) (end 170.0615 67.8615) (width 0.2) (layer "F.Cu") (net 10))
 (segment (start 170.0615 67.8615) (end 170 67.8) (width 0.2) (layer "F.Cu") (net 10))
 (segment (start 170 46.831374) (end 166.873126 43.7045) (width 0.2) (layer "F.Cu") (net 10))
 (segment (start 161.5 134.4) (end 170.0615 125.8385) (width 0.2) (layer "F.Cu") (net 10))
 (via (at 148.548 54.9275) (size 0.6) (drill 0.3) (layers "F.Cu" "B.Cu") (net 10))
 (segment (start 138.854 73.66) (end 138.854 73.5039) (width 0.2) (layer "F.Cu") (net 2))
 (segment (start 138.854 73.5039) (end 147.57895 64.77895) (width 0.2) (layer "F.Cu") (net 2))
 (segment (start 138.854 73.66) (end 152.714 59.8) (width 0.2) (layer "B.Cu") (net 2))
 (segment (start 152.714 59.8) (end 165.6 59.8) (width 0.2) (layer "B.Cu") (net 2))
 (segment (start 138.854 92.71) (end 166 65.564) (width 0.2) (layer "B.Cu") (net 9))
 (segment (start 166 65.564) (end 166 58.685) (width 0.2) (layer "B.Cu") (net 9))
 (segment (start 166 58.685) (end 164.7825 57.4675) (width 0.2) (layer "B.Cu") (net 9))
 (segment (start 139.434314 76.221628) (end 137.453 74.240314) (width 0.2) (layer "B.Cu") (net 17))
 (segment (start 137.453 88.18947) (end 139.434314 86.208156) (width 0.2) (layer "B.Cu") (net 17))
 (segment (start 139.434314 72.259) (end 156.765814 54.9275) (width 0.2) (layer "B.Cu") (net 17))
 (segment (start 156.765814 54.9275) (end 164.7825 54.9275) (width 0.2) (layer "B.Cu") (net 17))
 (segment (start 137.453 93.290314) (end 137.453 88.18947) (width 0.2) (layer "B.Cu") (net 17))
 (segment (start 139.434314 86.208156) (end 139.434314 76.221628) (width 0.2) (layer "B.Cu") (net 17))
 (segment (start 137.453 73.079686) (end 138.273686 72.259) (width 0.2) (layer "B.Cu") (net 17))
 (segment (start 138.854 94.691314) (end 137.453 93.290314) (width 0.2) (layer "B.Cu") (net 17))
 (segment (start 138.854 111.76) (end 138.854 94.691314) (width 0.2) (layer "B.Cu") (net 17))
 (segment (start 138.273686 72.259) (end 139.434314 72.259) (width 0.2) (layer "B.Cu") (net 17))
 (segment (start 137.453 74.240314) (end 137.453 73.079686) (width 0.2) (layer "B.Cu") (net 17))
 (segment (start 138.107586 71.858) (end 139.268214 71.858) (width 0.2) (layer "B.Cu") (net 6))
 (segment (start 139.268214 71.858) (end 158.738714 52.3875) (width 0.2) (layer "B.Cu") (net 6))
 (segment (start 158.738714 52.3875) (end 164.7825 52.3875) (width 0.2) (layer "B.Cu") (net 6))
 (segment (start 136.383 73.582586) (end 138.107586 71.858) (width 0.2) (layer "B.Cu") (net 6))
 (segment (start 136.383 128.339) (end 136.383 73.582586) (width 0.2) (layer "B.Cu") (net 6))
 (segment (start 138.854 130.81) (end 136.383 128.339) (width 0.2) (layer "B.Cu") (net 6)))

